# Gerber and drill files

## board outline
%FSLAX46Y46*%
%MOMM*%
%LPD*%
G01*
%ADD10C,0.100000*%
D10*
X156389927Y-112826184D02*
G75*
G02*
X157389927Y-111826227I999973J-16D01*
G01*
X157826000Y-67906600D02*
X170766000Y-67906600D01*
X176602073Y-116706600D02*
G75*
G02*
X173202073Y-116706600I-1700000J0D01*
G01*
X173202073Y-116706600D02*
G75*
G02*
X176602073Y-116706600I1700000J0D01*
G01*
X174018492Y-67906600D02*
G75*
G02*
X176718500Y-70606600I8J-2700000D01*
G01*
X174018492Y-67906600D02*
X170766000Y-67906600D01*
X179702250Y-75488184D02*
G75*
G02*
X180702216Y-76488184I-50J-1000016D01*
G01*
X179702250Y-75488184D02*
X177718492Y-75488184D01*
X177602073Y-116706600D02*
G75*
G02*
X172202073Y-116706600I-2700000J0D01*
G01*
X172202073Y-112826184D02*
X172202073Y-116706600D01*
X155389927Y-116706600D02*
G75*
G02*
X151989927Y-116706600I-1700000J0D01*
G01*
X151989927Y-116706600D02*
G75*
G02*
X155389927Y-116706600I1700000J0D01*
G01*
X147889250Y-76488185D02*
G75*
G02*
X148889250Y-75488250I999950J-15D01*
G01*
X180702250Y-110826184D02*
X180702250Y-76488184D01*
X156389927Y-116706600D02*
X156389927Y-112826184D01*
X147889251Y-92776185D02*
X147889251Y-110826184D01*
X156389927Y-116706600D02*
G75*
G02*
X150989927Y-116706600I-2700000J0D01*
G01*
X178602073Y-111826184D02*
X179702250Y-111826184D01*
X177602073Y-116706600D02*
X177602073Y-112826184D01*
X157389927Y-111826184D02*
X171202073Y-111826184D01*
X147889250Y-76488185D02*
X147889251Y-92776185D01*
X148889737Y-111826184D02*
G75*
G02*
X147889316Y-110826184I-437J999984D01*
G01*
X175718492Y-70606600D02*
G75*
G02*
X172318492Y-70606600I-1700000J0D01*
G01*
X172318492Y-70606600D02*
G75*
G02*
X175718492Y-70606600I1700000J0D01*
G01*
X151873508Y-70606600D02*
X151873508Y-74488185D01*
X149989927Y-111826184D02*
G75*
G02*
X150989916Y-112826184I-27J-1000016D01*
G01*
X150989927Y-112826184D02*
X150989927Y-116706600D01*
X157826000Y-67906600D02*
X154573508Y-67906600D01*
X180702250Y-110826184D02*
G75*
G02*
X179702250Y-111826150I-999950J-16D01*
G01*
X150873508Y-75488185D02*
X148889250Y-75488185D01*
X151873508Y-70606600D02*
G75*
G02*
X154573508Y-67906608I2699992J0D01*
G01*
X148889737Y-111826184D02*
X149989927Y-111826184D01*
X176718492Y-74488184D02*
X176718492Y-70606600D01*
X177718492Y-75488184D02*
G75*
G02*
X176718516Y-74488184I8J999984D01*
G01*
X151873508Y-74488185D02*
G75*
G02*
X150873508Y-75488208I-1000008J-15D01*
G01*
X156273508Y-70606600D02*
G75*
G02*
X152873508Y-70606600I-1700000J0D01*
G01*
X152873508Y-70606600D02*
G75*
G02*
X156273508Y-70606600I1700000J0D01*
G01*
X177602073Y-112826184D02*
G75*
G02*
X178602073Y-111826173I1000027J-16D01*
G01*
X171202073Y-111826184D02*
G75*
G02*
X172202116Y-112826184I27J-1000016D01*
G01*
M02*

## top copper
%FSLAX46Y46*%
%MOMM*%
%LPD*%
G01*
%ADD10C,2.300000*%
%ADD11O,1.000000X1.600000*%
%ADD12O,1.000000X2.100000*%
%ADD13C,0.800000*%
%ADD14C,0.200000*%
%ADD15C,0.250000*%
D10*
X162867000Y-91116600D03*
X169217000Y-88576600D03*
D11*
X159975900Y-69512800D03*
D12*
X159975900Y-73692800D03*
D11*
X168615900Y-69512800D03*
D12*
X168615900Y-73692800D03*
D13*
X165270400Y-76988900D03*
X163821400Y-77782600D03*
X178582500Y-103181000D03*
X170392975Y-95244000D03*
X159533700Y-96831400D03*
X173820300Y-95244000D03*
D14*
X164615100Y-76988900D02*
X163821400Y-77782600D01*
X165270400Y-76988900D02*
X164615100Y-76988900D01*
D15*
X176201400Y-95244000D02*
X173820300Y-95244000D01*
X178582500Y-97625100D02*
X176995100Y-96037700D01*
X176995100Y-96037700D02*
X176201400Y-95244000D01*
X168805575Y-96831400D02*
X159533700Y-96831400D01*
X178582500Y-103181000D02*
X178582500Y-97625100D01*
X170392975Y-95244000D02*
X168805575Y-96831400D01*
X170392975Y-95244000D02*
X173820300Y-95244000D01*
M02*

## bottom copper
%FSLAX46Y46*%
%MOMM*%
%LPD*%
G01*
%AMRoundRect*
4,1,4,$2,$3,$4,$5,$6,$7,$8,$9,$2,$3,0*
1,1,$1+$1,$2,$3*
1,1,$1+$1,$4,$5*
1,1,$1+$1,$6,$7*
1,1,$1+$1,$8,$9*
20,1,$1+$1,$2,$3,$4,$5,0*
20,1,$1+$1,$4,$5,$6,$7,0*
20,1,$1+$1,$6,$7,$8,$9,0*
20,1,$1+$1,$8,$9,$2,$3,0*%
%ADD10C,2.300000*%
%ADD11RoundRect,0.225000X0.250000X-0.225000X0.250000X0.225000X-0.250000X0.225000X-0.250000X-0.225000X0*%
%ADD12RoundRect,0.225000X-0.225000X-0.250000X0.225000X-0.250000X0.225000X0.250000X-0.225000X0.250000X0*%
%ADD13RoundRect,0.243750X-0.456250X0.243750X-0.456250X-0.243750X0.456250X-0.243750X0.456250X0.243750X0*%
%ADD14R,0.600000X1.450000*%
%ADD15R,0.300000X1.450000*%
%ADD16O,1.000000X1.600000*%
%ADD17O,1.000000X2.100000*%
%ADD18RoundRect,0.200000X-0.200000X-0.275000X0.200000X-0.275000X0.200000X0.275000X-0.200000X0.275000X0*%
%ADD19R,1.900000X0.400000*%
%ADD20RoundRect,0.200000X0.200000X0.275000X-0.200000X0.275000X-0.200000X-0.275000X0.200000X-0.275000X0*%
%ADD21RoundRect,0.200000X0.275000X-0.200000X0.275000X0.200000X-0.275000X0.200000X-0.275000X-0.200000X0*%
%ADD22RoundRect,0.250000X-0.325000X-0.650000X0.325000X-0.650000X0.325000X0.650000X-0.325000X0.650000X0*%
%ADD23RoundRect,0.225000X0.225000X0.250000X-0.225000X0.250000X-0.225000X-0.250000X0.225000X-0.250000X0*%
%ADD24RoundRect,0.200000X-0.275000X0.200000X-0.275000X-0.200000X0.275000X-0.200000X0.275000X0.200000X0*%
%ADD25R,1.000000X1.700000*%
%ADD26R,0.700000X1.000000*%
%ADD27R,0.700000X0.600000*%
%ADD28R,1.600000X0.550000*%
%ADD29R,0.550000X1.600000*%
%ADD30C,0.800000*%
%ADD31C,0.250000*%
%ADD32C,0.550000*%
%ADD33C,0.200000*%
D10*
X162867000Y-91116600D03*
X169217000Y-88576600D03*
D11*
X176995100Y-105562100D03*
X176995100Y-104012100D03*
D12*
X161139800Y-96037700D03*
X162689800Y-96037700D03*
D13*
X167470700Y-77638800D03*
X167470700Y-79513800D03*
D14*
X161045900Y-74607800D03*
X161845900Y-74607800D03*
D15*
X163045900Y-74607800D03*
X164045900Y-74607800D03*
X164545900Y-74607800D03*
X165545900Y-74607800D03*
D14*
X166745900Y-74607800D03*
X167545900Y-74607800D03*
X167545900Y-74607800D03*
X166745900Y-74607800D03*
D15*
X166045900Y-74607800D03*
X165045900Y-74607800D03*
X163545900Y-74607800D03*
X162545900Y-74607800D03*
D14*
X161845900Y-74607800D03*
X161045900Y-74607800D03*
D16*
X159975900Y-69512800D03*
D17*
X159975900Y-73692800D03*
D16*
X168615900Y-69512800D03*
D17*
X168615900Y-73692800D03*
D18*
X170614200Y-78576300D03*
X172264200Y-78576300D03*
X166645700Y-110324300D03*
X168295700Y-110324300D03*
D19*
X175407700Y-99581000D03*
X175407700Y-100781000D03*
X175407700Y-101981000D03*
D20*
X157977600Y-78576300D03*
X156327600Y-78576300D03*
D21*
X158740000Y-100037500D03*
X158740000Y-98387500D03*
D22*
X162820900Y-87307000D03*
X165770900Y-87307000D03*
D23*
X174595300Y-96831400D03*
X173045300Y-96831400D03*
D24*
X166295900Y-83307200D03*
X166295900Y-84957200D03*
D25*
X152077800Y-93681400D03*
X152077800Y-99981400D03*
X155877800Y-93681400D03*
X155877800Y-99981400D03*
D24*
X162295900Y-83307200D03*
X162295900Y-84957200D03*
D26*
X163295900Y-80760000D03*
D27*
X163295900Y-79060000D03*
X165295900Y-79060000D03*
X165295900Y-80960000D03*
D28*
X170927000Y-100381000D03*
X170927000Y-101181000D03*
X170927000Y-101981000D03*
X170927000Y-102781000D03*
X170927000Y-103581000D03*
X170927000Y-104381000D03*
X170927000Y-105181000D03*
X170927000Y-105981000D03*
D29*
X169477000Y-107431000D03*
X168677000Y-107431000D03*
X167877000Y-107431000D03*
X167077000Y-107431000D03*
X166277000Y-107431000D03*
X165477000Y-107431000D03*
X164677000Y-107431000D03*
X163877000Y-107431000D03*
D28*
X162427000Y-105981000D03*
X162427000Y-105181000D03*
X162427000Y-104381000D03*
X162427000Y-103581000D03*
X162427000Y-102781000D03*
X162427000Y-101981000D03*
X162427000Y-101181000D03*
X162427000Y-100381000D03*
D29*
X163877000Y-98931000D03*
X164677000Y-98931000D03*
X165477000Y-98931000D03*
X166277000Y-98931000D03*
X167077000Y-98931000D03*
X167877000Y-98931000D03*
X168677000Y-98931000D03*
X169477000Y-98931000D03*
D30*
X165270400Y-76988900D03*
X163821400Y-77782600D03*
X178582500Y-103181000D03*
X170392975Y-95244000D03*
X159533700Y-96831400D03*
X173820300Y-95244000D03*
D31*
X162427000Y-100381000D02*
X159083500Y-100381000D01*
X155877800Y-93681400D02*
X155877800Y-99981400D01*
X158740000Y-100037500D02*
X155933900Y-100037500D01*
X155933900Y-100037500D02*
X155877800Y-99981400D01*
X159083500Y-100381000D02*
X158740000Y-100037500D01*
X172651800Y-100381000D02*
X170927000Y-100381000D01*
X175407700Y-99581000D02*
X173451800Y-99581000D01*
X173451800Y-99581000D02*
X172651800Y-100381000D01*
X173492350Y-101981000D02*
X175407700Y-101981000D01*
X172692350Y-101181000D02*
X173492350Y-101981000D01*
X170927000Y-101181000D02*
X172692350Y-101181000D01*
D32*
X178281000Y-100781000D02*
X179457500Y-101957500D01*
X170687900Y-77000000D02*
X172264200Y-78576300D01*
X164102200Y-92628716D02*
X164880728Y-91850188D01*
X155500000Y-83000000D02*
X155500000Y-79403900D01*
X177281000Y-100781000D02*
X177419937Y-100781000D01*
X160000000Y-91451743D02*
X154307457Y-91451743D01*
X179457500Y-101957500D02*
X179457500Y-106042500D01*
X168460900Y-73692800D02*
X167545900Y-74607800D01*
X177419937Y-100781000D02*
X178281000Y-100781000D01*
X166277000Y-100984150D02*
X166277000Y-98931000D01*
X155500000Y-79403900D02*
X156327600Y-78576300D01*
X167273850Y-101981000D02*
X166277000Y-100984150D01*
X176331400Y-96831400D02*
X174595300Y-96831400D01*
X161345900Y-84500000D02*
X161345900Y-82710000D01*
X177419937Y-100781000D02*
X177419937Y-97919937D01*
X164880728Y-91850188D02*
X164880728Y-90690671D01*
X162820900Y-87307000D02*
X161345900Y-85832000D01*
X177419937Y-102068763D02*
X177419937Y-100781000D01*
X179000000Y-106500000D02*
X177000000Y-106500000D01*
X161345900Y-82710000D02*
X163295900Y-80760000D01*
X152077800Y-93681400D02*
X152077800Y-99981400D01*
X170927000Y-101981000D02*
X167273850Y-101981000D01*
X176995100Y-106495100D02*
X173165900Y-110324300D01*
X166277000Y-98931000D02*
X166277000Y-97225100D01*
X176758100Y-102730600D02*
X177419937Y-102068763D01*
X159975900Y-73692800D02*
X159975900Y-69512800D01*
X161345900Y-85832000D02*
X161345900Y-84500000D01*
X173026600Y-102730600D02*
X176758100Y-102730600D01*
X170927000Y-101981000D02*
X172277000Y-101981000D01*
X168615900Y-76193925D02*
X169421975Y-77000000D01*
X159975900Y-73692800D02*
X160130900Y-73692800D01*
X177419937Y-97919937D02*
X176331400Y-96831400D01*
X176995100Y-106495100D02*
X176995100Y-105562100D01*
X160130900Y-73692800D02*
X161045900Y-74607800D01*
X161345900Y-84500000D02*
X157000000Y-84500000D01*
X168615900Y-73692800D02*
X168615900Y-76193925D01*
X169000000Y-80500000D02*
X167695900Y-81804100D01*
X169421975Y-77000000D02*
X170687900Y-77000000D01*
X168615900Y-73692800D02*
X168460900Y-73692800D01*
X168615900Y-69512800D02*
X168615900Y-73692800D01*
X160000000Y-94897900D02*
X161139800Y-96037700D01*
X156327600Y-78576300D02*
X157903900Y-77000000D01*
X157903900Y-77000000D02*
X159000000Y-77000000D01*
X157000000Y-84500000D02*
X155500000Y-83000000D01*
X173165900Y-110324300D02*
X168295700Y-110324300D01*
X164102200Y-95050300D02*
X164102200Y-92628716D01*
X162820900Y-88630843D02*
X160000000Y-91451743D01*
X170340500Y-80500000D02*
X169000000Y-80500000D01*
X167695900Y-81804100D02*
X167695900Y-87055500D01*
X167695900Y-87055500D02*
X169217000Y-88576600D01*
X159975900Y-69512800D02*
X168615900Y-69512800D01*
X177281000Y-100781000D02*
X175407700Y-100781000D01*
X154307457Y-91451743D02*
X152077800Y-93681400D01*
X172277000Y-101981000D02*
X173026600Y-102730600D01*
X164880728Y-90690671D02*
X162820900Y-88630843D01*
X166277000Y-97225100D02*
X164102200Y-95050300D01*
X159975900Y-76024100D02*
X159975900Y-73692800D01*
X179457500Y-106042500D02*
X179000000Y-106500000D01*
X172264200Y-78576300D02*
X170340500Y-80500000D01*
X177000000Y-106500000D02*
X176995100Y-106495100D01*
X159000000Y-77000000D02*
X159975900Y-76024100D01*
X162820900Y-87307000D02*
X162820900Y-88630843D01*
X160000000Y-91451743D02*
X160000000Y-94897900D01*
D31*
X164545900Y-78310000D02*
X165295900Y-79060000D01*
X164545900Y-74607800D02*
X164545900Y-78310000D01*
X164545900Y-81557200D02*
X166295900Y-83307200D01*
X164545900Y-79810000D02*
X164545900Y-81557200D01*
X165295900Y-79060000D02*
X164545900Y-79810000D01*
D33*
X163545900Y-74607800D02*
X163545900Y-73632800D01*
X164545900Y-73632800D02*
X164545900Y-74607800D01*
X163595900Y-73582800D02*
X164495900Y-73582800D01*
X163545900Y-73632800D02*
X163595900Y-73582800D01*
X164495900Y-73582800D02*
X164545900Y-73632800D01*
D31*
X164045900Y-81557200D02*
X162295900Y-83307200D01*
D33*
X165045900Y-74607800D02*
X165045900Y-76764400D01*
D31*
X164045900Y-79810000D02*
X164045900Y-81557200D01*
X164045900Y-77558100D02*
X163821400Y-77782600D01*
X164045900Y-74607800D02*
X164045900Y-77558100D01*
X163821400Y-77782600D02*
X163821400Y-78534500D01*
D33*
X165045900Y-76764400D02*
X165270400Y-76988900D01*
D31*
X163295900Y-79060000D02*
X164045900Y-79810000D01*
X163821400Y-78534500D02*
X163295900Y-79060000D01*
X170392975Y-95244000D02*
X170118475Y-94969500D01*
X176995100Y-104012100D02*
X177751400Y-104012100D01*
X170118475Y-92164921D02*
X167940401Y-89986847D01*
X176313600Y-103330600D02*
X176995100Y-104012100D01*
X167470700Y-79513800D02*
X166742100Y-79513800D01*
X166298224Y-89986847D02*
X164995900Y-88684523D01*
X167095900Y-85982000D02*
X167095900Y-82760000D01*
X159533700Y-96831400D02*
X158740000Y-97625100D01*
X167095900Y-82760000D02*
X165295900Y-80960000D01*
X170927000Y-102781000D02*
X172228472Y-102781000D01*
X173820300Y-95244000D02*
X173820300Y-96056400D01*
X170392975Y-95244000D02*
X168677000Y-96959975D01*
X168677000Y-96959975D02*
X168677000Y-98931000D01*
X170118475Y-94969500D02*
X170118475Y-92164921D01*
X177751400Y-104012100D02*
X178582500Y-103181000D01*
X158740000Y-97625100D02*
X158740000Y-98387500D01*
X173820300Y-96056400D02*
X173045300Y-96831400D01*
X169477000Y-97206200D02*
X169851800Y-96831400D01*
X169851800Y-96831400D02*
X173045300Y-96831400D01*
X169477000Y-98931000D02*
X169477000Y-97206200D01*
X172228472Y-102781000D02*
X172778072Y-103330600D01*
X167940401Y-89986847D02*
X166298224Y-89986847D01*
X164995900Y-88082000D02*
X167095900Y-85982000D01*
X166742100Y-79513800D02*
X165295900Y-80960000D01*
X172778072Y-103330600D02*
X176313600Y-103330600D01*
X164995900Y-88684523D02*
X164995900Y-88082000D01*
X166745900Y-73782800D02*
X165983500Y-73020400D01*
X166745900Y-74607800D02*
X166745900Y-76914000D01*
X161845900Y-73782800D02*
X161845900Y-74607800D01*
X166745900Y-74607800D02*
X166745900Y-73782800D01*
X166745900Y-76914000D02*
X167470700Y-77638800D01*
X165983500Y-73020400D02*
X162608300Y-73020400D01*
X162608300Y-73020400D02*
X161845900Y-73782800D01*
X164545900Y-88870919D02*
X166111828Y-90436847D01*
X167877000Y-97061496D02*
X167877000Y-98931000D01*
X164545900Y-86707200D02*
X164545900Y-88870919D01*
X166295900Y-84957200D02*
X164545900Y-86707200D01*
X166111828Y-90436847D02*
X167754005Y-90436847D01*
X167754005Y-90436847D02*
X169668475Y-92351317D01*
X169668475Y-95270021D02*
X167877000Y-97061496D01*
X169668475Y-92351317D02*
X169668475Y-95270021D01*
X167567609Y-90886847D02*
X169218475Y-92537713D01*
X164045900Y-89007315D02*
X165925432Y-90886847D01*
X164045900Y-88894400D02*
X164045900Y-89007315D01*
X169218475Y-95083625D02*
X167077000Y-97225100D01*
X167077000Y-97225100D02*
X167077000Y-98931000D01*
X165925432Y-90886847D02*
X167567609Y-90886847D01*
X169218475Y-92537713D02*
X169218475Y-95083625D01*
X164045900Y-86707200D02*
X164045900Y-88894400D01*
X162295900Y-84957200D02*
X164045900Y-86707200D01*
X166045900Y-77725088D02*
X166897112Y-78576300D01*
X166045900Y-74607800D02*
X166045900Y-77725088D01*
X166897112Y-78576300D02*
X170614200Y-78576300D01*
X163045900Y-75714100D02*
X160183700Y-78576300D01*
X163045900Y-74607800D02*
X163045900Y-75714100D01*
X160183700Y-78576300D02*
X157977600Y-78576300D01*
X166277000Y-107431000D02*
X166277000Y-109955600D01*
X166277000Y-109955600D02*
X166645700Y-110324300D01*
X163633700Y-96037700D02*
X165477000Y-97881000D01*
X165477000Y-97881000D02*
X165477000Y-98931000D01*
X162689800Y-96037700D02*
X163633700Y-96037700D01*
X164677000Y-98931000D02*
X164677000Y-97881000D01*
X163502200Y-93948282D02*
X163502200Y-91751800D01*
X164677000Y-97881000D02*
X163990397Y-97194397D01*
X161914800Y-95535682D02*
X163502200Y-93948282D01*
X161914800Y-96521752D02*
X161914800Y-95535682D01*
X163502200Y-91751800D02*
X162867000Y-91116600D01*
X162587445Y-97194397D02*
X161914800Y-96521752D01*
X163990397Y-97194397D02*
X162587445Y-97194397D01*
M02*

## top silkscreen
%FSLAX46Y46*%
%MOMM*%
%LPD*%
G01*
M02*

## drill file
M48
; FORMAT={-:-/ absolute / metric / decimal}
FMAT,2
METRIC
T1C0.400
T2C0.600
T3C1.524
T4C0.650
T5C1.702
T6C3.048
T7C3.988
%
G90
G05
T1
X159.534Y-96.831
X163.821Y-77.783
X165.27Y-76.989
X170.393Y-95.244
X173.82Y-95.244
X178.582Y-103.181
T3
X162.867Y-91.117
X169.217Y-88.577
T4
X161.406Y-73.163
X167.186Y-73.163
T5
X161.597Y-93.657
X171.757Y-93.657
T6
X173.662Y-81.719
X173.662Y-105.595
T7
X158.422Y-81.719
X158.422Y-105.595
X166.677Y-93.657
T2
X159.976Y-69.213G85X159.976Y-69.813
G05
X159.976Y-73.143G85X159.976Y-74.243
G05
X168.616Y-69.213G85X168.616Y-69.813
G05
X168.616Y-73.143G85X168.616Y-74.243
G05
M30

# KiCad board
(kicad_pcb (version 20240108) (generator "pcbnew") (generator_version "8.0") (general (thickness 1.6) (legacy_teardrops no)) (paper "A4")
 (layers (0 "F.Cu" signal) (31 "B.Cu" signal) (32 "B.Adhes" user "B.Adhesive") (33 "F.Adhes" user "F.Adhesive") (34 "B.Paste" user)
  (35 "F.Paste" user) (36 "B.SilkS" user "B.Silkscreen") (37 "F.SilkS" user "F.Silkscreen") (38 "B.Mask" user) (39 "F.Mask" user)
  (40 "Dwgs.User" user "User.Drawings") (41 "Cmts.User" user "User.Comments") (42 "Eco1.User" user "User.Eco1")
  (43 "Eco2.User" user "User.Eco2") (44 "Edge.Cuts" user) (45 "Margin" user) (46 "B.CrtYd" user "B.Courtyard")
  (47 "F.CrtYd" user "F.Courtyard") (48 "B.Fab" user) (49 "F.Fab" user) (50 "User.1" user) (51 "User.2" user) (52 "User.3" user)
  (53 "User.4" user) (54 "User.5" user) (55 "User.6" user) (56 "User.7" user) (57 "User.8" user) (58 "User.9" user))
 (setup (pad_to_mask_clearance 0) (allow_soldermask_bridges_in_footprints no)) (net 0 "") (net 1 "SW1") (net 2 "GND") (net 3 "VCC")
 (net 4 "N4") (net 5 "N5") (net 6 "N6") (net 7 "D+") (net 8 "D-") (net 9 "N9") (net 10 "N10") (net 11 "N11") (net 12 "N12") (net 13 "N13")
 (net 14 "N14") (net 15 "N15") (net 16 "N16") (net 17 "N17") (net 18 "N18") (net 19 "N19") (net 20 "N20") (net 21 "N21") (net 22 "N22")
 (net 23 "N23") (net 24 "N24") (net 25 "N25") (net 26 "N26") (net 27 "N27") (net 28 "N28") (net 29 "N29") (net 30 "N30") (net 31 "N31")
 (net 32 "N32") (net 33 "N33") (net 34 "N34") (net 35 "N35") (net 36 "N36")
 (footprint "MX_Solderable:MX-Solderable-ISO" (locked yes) (layer "F.Cu") (at 166.677 93.6566)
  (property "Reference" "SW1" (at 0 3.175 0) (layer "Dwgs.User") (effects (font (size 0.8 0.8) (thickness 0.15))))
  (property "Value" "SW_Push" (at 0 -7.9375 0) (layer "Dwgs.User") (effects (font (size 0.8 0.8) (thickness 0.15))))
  (pad "" np_thru_hole circle (at -8.255 -11.938) (size 3.9878 3.9878) (drill 3.9878) (layers "*.Cu" "*.Mask"))
  (pad "" np_thru_hole circle (at -8.255 11.938) (size 3.9878 3.9878) (drill 3.9878) (layers "*.Cu" "*.Mask"))
  (pad "" np_thru_hole circle (at -5.08 0 48.099) (size 1.7018 1.7018) (drill 1.7018) (layers "F&B.Cu" "*.Mask"))
  (pad "" np_thru_hole circle (at 0 0) (size 3.9878 3.9878) (drill 3.9878) (layers "*.Cu" "*.Mask"))
  (pad "" np_thru_hole circle (at 5.08 0 48.099) (size 1.7018 1.7018) (drill 1.7018) (layers "F&B.Cu" "*.Mask"))
  (pad "" np_thru_hole circle (at 6.985 -11.938) (size 3.048 3.048) (drill 3.048) (layers "*.Cu" "*.Mask"))
  (pad "" np_thru_hole circle (at 6.985 11.938) (size 3.048 3.048) (drill 3.048) (layers "*.Cu" "*.Mask"))
  (pad "1" thru_hole circle (at -3.81 -2.54) (size 2.3 2.3) (drill 1.524) (layers "*.Cu" "B.Mask") (remove_unused_layers no) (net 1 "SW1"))
  (pad "2" thru_hole circle (at 2.54 -5.08) (size 2.3 2.3) (drill 1.524) (layers "*.Cu" "B.Mask") (remove_unused_layers no) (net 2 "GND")))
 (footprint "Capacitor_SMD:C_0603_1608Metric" (layer "B.Cu") (at 176.9951 104.7871 90)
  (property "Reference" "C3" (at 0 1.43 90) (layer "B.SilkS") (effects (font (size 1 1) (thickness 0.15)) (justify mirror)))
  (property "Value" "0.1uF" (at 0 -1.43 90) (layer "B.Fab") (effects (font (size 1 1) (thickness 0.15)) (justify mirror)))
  (pad "1" smd roundrect (at -0.775 0 90) (size 0.9 0.95) (layers "B.Cu" "B.Paste" "B.Mask") (roundrect_rratio 0.25) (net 2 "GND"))
  (pad "2" smd roundrect (at 0.775 0 90) (size 0.9 0.95) (layers "B.Cu" "B.Paste" "B.Mask") (roundrect_rratio 0.25) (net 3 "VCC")))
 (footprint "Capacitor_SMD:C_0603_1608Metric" (layer "B.Cu") (at 161.9148 96.0377)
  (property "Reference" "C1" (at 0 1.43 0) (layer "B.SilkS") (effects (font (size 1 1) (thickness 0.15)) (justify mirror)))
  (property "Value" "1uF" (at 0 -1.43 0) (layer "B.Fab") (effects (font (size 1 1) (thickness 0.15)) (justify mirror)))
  (pad "1" smd roundrect (at -0.775 0) (size 0.9 0.95) (layers "B.Cu" "B.Paste" "B.Mask") (roundrect_rratio 0.25) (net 2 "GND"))
  (pad "2" smd roundrect (at 0.775 0) (size 0.9 0.95) (layers "B.Cu" "B.Paste" "B.Mask") (roundrect_rratio 0.25) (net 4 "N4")))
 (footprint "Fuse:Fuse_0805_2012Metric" (layer "B.Cu") (at 167.4707 78.5763 -90)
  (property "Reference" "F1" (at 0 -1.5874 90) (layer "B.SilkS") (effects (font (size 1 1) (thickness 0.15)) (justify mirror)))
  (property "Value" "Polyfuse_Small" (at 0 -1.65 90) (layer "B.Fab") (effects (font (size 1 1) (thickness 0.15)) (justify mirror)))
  (pad "1" smd roundrect (at -0.9375 0 270) (size 0.975 1.4) (layers "B.Cu" "B.Paste" "B.Mask") (roundrect_rratio 0.25) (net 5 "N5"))
  (pad "2" smd roundrect (at 0.9375 0 270) (size 0.975 1.4) (layers "B.Cu" "B.Paste" "B.Mask") (roundrect_rratio 0.25) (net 3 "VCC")))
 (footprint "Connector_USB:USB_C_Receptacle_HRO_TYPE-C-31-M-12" (layer "B.Cu") (at 164.2959 70.5628)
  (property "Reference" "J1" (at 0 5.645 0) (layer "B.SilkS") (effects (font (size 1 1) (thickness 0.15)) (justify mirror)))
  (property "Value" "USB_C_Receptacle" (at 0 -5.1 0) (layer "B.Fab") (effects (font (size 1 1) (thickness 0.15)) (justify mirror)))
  (pad "" np_thru_hole circle (at -2.89 2.6) (size 0.65 0.65) (drill 0.65) (layers "*.Cu" "*.Mask"))
  (pad "" np_thru_hole circle (at 2.89 2.6) (size 0.65 0.65) (drill 0.65) (layers "*.Cu" "*.Mask"))
  (pad "A1" smd rect (at -3.25 4.045) (size 0.6 1.45) (layers "B.Cu" "B.Paste" "B.Mask") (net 2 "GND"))
  (pad "A4" smd rect (at -2.45 4.045) (size 0.6 1.45) (layers "B.Cu" "B.Paste" "B.Mask") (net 5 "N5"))
  (pad "A5" smd rect (at -1.25 4.045) (size 0.3 1.45) (layers "B.Cu" "B.Paste" "B.Mask") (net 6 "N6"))
  (pad "A6" smd rect (at -0.25 4.045) (size 0.3 1.45) (layers "B.Cu" "B.Paste" "B.Mask") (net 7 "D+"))
  (pad "A7" smd rect (at 0.25 4.045) (size 0.3 1.45) (layers "B.Cu" "B.Paste" "B.Mask") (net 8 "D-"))
  (pad "A8" smd rect (at 1.25 4.045) (size 0.3 1.45) (layers "B.Cu" "B.Paste" "B.Mask") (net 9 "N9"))
  (pad "A9" smd rect (at 2.45 4.045) (size 0.6 1.45) (layers "B.Cu" "B.Paste" "B.Mask") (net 5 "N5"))
  (pad "A12" smd rect (at 3.25 4.045) (size 0.6 1.45) (layers "B.Cu" "B.Paste" "B.Mask") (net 2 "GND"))
  (pad "B1" smd rect (at 3.25 4.045) (size 0.6 1.45) (layers "B.Cu" "B.Paste" "B.Mask") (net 2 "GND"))
  (pad "B4" smd rect (at 2.45 4.045) (size 0.6 1.45) (layers "B.Cu" "B.Paste" "B.Mask") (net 5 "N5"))
  (pad "B5" smd rect (at 1.75 4.045) (size 0.3 1.45) (layers "B.Cu" "B.Paste" "B.Mask") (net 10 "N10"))
  (pad "B6" smd rect (at 0.75 4.045) (size 0.3 1.45) (layers "B.Cu" "B.Paste" "B.Mask") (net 7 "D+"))
  (pad "B7" smd rect (at -0.75 4.045) (size 0.3 1.45) (layers "B.Cu" "B.Paste" "B.Mask") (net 8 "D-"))
  (pad "B8" smd rect (at -1.75 4.045) (size 0.3 1.45) (layers "B.Cu" "B.Paste" "B.Mask") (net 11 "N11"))
  (pad "B9" smd rect (at -2.45 4.045) (size 0.6 1.45) (layers "B.Cu" "B.Paste" "B.Mask") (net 5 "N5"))
  (pad "B12" smd rect (at -3.25 4.045) (size 0.6 1.45) (layers "B.Cu" "B.Paste" "B.Mask") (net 2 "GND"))
  (pad "S1" thru_hole oval (at -4.32 -1.05) (size 1 1.6) (drill oval 0.6 1.2) (layers "*.Cu" "*.Mask") (remove_unused_layers no)
   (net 2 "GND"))
  (pad "S1" thru_hole oval (at -4.32 3.13) (size 1 2.1) (drill oval 0.6 1.7) (layers "*.Cu" "*.Mask") (remove_unused_layers no)
   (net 2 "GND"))
  (pad "S1" thru_hole oval (at 4.32 -1.05) (size 1 1.6) (drill oval 0.6 1.2) (layers "*.Cu" "*.Mask") (remove_unused_layers no)
   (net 2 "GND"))
  (pad "S1" thru_hole oval (at 4.32 3.13) (size 1 2.1) (drill oval 0.6 1.7) (layers "*.Cu" "*.Mask") (remove_unused_layers no) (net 2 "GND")))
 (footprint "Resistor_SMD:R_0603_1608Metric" (layer "B.Cu") (at 171.4392 78.5763)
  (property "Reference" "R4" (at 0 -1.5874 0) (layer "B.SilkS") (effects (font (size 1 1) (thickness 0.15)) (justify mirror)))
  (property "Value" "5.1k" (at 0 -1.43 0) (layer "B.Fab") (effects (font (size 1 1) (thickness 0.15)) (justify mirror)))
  (pad "1" smd roundrect (at -0.825 0) (size 0.8 0.95) (layers "B.Cu" "B.Paste" "B.Mask") (roundrect_rratio 0.25) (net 10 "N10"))
  (pad "2" smd roundrect (at 0.825 0) (size 0.8 0.95) (layers "B.Cu" "B.Paste" "B.Mask") (roundrect_rratio 0.25) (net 2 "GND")))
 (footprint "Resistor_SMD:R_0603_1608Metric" (layer "B.Cu") (at 167.4707 110.3243)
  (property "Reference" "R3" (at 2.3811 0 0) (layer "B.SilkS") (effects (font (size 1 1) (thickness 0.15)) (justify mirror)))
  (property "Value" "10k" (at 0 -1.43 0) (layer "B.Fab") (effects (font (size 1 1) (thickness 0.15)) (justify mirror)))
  (pad "1" smd roundrect (at -0.825 0) (size 0.8 0.95) (layers "B.Cu" "B.Paste" "B.Mask") (roundrect_rratio 0.25) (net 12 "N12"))
  (pad "2" smd roundrect (at 0.825 0) (size 0.8 0.95) (layers "B.Cu" "B.Paste" "B.Mask") (roundrect_rratio 0.25) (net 2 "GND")))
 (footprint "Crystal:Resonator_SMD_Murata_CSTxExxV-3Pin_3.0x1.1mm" (layer "B.Cu") (at 175.4077 100.781 -90)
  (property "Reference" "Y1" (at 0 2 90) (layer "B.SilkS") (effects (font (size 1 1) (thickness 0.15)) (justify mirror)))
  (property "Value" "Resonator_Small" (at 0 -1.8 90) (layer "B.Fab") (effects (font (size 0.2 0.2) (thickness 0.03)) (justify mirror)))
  (pad "1" smd rect (at -1.2 0 270) (size 0.4 1.9) (layers "B.Cu" "B.Paste" "B.Mask") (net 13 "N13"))
  (pad "2" smd rect (at 0 0 270) (size 0.4 1.9) (layers "B.Cu" "B.Paste" "B.Mask") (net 2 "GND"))
  (pad "3" smd rect (at 1.2 0 270) (size 0.4 1.9) (layers "B.Cu" "B.Paste" "B.Mask") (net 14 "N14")))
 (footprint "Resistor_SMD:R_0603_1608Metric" (layer "B.Cu") (at 157.1526 78.5763 180)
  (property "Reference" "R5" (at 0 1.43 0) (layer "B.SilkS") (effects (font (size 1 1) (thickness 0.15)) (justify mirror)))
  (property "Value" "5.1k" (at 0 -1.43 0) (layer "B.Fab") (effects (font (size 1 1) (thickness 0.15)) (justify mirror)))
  (pad "1" smd roundrect (at -0.825 0 180) (size 0.8 0.95) (layers "B.Cu" "B.Paste" "B.Mask") (roundrect_rratio 0.25) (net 6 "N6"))
  (pad "2" smd roundrect (at 0.825 0 180) (size 0.8 0.95) (layers "B.Cu" "B.Paste" "B.Mask") (roundrect_rratio 0.25) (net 2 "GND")))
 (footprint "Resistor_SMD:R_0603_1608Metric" (layer "B.Cu") (at 158.74 99.2125 90)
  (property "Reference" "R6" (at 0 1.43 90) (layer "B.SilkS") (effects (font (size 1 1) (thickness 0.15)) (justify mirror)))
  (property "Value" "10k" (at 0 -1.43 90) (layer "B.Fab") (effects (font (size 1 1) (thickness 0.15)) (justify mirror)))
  (pad "1" smd roundrect (at -0.825 0 90) (size 0.8 0.95) (layers "B.Cu" "B.Paste" "B.Mask") (roundrect_rratio 0.25) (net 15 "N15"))
  (pad "2" smd roundrect (at 0.825 0 90) (size 0.8 0.95) (layers "B.Cu" "B.Paste" "B.Mask") (roundrect_rratio 0.25) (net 3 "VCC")))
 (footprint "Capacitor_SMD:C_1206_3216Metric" (layer "B.Cu") (at 164.2959 87.307)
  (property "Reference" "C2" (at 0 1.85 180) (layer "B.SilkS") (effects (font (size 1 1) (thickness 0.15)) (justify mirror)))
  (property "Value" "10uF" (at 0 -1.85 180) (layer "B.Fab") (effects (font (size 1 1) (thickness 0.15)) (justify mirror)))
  (pad "1" smd roundrect (at -1.475 0) (size 1.15 1.8) (layers "B.Cu" "B.Paste" "B.Mask") (roundrect_rratio 0.2173913043) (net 2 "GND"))
  (pad "2" smd roundrect (at 1.475 0) (size 1.15 1.8) (layers "B.Cu" "B.Paste" "B.Mask") (roundrect_rratio 0.2173913043) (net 3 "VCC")))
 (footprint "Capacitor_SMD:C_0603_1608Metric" (layer "B.Cu") (at 173.8203 96.8314 180)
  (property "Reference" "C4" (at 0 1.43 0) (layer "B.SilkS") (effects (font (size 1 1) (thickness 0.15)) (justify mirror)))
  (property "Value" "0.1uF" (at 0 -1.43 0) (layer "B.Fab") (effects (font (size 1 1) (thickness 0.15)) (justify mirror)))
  (pad "1" smd roundrect (at -0.775 0 180) (size 0.9 0.95) (layers "B.Cu" "B.Paste" "B.Mask") (roundrect_rratio 0.25) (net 2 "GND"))
  (pad "2" smd roundrect (at 0.775 0 180) (size 0.9 0.95) (layers "B.Cu" "B.Paste" "B.Mask") (roundrect_rratio 0.25) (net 3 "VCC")))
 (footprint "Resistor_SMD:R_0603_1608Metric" (layer "B.Cu") (at 166.2959 84.1322 -90)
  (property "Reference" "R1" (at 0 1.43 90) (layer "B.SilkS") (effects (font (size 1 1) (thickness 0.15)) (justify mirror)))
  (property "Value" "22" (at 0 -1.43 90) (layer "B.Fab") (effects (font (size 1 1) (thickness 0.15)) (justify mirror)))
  (pad "1" smd roundrect (at -0.825 0 270) (size 0.8 0.95) (layers "B.Cu" "B.Paste" "B.Mask") (roundrect_rratio 0.25) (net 8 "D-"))
  (pad "2" smd roundrect (at 0.825 0 270) (size 0.8 0.95) (layers "B.Cu" "B.Paste" "B.Mask") (roundrect_rratio 0.25) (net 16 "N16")))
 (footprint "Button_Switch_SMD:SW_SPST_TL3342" (layer "B.Cu") (at 153.9778 96.8314 -90)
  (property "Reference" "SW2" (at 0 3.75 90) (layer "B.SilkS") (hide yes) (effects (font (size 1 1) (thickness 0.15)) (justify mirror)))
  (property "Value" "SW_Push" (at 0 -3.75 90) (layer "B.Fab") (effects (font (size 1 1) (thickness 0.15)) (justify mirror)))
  (pad "1" smd rect (at -3.15 1.9 270) (size 1.7 1) (layers "B.Cu" "B.Paste" "B.Mask") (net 2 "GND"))
  (pad "1" smd rect (at 3.15 1.9 270) (size 1.7 1) (layers "B.Cu" "B.Paste" "B.Mask") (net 2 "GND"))
  (pad "2" smd rect (at -3.15 -1.9 270) (size 1.7 1) (layers "B.Cu" "B.Paste" "B.Mask") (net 15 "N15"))
  (pad "2" smd rect (at 3.15 -1.9 270) (size 1.7 1) (layers "B.Cu" "B.Paste" "B.Mask") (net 15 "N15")))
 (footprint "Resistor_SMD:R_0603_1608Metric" (layer "B.Cu") (at 162.2959 84.1322 -90)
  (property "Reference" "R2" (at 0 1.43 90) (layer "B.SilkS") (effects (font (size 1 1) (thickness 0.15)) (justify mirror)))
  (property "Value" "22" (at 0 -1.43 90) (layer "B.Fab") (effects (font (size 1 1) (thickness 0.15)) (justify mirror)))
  (pad "1" smd roundrect (at -0.825 0 270) (size 0.8 0.95) (layers "B.Cu" "B.Paste" "B.Mask") (roundrect_rratio 0.25) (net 7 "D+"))
  (pad "2" smd roundrect (at 0.825 0 270) (size 0.8 0.95) (layers "B.Cu" "B.Paste" "B.Mask") (roundrect_rratio 0.25) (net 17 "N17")))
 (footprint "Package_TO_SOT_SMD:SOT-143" (layer "B.Cu") (at 164.2959 80.01)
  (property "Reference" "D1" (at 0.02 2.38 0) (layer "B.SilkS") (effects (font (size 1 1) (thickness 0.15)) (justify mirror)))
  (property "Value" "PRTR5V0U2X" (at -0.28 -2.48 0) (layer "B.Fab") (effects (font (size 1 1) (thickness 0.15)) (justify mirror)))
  (pad "1" smd rect (at -1 0.75) (size 0.7 1) (layers "B.Cu" "B.Paste" "B.Mask") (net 2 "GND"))
  (pad "2" smd rect (at -1 -0.95) (size 0.7 0.6) (layers "B.Cu" "B.Paste" "B.Mask") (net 7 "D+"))
  (pad "3" smd rect (at 1 -0.95) (size 0.7 0.6) (layers "B.Cu" "B.Paste" "B.Mask") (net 8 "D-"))
  (pad "4" smd rect (at 1 0.95) (size 0.7 0.6) (layers "B.Cu" "B.Paste" "B.Mask") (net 3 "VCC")))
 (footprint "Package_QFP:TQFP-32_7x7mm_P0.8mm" (layer "B.Cu") (at 166.677 103.181 180)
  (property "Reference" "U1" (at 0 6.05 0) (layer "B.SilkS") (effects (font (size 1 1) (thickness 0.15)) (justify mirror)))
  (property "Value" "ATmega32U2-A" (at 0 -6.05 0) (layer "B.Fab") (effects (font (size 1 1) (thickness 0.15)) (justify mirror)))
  (pad "1" smd rect (at -4.25 2.8 180) (size 1.6 0.55) (layers "B.Cu" "B.Paste" "B.Mask") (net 13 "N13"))
  (pad "2" smd rect (at -4.25 2 180) (size 1.6 0.55) (layers "B.Cu" "B.Paste" "B.Mask") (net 14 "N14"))
  (pad "3" smd rect (at -4.25 1.2 180) (size 1.6 0.55) (layers "B.Cu" "B.Paste" "B.Mask") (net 2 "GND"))
  (pad "4" smd rect (at -4.25 0.4 180) (size 1.6 0.55) (layers "B.Cu" "B.Paste" "B.Mask") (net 3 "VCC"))
  (pad "5" smd rect (at -4.25 -0.4 180) (size 1.6 0.55) (layers "B.Cu" "B.Paste" "B.Mask") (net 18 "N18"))
  (pad "6" smd rect (at -4.25 -1.2 180) (size 1.6 0.55) (layers "B.Cu" "B.Paste" "B.Mask") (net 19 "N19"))
  (pad "7" smd rect (at -4.25 -2 180) (size 1.6 0.55) (layers "B.Cu" "B.Paste" "B.Mask") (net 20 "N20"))
  (pad "8" smd rect (at -4.25 -2.8 180) (size 1.6 0.55) (layers "B.Cu" "B.Paste" "B.Mask") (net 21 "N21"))
  (pad "9" smd rect (at -2.8 -4.25 90) (size 1.6 0.55) (layers "B.Cu" "B.Paste" "B.Mask") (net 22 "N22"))
  (pad "10" smd rect (at -2 -4.25 90) (size 1.6 0.55) (layers "B.Cu" "B.Paste" "B.Mask") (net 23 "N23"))
  (pad "11" smd rect (at -1.2 -4.25 90) (size 1.6 0.55) (layers "B.Cu" "B.Paste" "B.Mask") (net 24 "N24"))
  (pad "12" smd rect (at -0.4 -4.25 90) (size 1.6 0.55) (layers "B.Cu" "B.Paste" "B.Mask") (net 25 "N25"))
  (pad "13" smd rect (at 0.4 -4.25 90) (size 1.6 0.55) (layers "B.Cu" "B.Paste" "B.Mask") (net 12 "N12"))
  (pad "14" smd rect (at 1.2 -4.25 90) (size 1.6 0.55) (layers "B.Cu" "B.Paste" "B.Mask") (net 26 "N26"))
  (pad "15" smd rect (at 2 -4.25 90) (size 1.6 0.55) (layers "B.Cu" "B.Paste" "B.Mask") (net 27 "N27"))
  (pad "16" smd rect (at 2.8 -4.25 90) (size 1.6 0.55) (layers "B.Cu" "B.Paste" "B.Mask") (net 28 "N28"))
  (pad "17" smd rect (at 4.25 -2.8 180) (size 1.6 0.55) (layers "B.Cu" "B.Paste" "B.Mask") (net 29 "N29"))
  (pad "18" smd rect (at 4.25 -2 180) (size 1.6 0.55) (layers "B.Cu" "B.Paste" "B.Mask") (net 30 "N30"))
  (pad "19" smd rect (at 4.25 -1.2 180) (size 1.6 0.55) (layers "B.Cu" "B.Paste" "B.Mask") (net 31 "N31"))
  (pad "20" smd rect (at 4.25 -0.4 180) (size 1.6 0.55) (layers "B.Cu" "B.Paste" "B.Mask") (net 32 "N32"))
  (pad "21" smd rect (at 4.25 0.4 180) (size 1.6 0.55) (layers "B.Cu" "B.Paste" "B.Mask") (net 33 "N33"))
  (pad "22" smd rect (at 4.25 1.2 180) (size 1.6 0.55) (layers "B.Cu" "B.Paste" "B.Mask") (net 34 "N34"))
  (pad "23" smd rect (at 4.25 2 180) (size 1.6 0.55) (layers "B.Cu" "B.Paste" "B.Mask") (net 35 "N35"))
  (pad "24" smd rect (at 4.25 2.8 180) (size 1.6 0.55) (layers "B.Cu" "B.Paste" "B.Mask") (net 15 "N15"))
  (pad "25" smd rect (at 2.8 4.25 90) (size 1.6 0.55) (layers "B.Cu" "B.Paste" "B.Mask") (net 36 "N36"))
  (pad "26" smd rect (at 2 4.25 90) (size 1.6 0.55) (layers "B.Cu" "B.Paste" "B.Mask") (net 1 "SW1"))
  (pad "27" smd rect (at 1.2 4.25 90) (size 1.6 0.55) (layers "B.Cu" "B.Paste" "B.Mask") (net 4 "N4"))
  (pad "28" smd rect (at 0.4 4.25 90) (size 1.6 0.55) (layers "B.Cu" "B.Paste" "B.Mask") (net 2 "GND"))
  (pad "29" smd rect (at -0.4 4.25 90) (size 1.6 0.55) (layers "B.Cu" "B.Paste" "B.Mask") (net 17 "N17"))
  (pad "30" smd rect (at -1.2 4.25 90) (size 1.6 0.55) (layers "B.Cu" "B.Paste" "B.Mask") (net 16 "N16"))
  (pad "31" smd rect (at -2 4.25 90) (size 1.6 0.55) (layers "B.Cu" "B.Paste" "B.Mask") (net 3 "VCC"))
  (pad "32" smd rect (at -2.8 4.25 90) (size 1.6 0.55) (layers "B.Cu" "B.Paste" "B.Mask") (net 3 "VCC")))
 (gr_arc (start 156.389927 112.826184) (mid 156.682821 112.119078) (end 157.389927 111.826184) (stroke (width 0.1) (type solid))
  (layer "Edge.Cuts"))
 (gr_line (start 157.826 67.9066) (end 170.766 67.9066) (stroke (width 0.1) (type default)) (layer "Edge.Cuts"))
 (gr_circle (center 174.902073 116.7066) (end 173.202073 116.7066) (stroke (width 0.1) (type solid)) (fill none) (layer "Edge.Cuts"))
 (gr_arc (start 174.018492 67.9066) (mid 175.92768 68.697412) (end 176.718492 70.6066) (stroke (width 0.1) (type solid)) (layer "Edge.Cuts"))
 (gr_line (start 174.018492 67.9066) (end 170.766 67.9066) (stroke (width 0.1) (type solid)) (layer "Edge.Cuts"))
 (gr_arc (start 179.70225 75.488184) (mid 180.409356 75.781078) (end 180.70225 76.488184) (stroke (width 0.1) (type solid))
  (layer "Edge.Cuts"))
 (gr_line (start 179.70225 75.488184) (end 177.718492 75.488184) (stroke (width 0.1) (type solid)) (layer "Edge.Cuts"))
 (gr_arc (start 177.602073 116.7066) (mid 174.902073 119.4066) (end 172.202073 116.7066) (stroke (width 0.1) (type solid))
  (layer "Edge.Cuts"))
 (gr_line (start 172.202073 112.826184) (end 172.202073 116.7066) (stroke (width 0.1) (type solid)) (layer "Edge.Cuts"))
 (gr_circle (center 153.689927 116.7066) (end 151.989927 116.7066) (stroke (width 0.1) (type solid)) (fill none) (layer "Edge.Cuts"))
 (gr_arc (start 147.88925 76.488185) (mid 148.182141 75.781075) (end 148.88925 75.488185) (stroke (width 0.1) (type solid))
  (layer "Edge.Cuts"))
 (gr_line (start 180.70225 110.826184) (end 180.70225 76.488184) (stroke (width 0.1) (type solid)) (layer "Edge.Cuts"))
 (gr_line (start 156.389927 116.7066) (end 156.389927 112.826184) (stroke (width 0.1) (type solid)) (layer "Edge.Cuts"))
 (gr_line (start 147.889251 92.776185) (end 147.889251 110.826184) (stroke (width 0.1) (type solid)) (layer "Edge.Cuts"))
 (gr_arc (start 156.389927 116.7066) (mid 153.689927 119.4066) (end 150.989927 116.7066) (stroke (width 0.1) (type solid))
  (layer "Edge.Cuts"))
 (gr_line (start 178.602073 111.826184) (end 179.70225 111.826184) (stroke (width 0.1) (type solid)) (layer "Edge.Cuts"))
 (gr_line (start 177.602073 116.7066) (end 177.602073 112.826184) (stroke (width 0.1) (type solid)) (layer "Edge.Cuts"))
 (gr_line (start 157.389927 111.826184) (end 171.202073 111.826184) (stroke (width 0.1) (type solid)) (layer "Edge.Cuts"))
 (gr_line (start 147.88925 76.488185) (end 147.889251 92.776185) (stroke (width 0.1) (type solid)) (layer "Edge.Cuts"))
 (gr_arc (start 148.889737 111.826184) (mid 148.182316 111.533463) (end 147.889251 110.826184) (stroke (width 0.1) (type solid))
  (layer "Edge.Cuts"))
 (gr_circle (center 174.018492 70.6066) (end 172.318492 70.6066) (stroke (width 0.1) (type solid)) (fill none) (layer "Edge.Cuts"))
 (gr_line (start 151.873508 70.6066) (end 151.873508 74.488185) (stroke (width 0.1) (type solid)) (layer "Edge.Cuts"))
 (gr_arc (start 149.989927 111.826184) (mid 150.697033 112.119078) (end 150.989927 112.826184) (stroke (width 0.1) (type solid))
  (layer "Edge.Cuts"))
 (gr_line (start 150.989927 112.826184) (end 150.989927 116.7066) (stroke (width 0.1) (type solid)) (layer "Edge.Cuts"))
 (gr_line (start 157.826 67.9066) (end 154.573508 67.9066) (stroke (width 0.1) (type solid)) (layer "Edge.Cuts"))
 (gr_arc (start 180.70225 110.826184) (mid 180.409357 111.533291) (end 179.70225 111.826184) (stroke (width 0.1) (type solid))
  (layer "Edge.Cuts"))
 (gr_line (start 150.873508 75.488185) (end 148.88925 75.488185) (stroke (width 0.1) (type solid)) (layer "Edge.Cuts"))
 (gr_arc (start 151.873508 70.6066) (mid 152.66432 68.697412) (end 154.573508 67.9066) (stroke (width 0.1) (type solid)) (layer "Edge.Cuts"))
 (gr_line (start 148.889737 111.826184) (end 149.989927 111.826184) (stroke (width 0.1) (type solid)) (layer "Edge.Cuts"))
 (gr_line (start 176.718492 74.488184) (end 176.718492 70.6066) (stroke (width 0.1) (type solid)) (layer "Edge.Cuts"))
 (gr_arc (start 177.718492 75.488184) (mid 177.011385 75.195291) (end 176.718492 74.488184) (stroke (width 0.1) (type solid))
  (layer "Edge.Cuts"))
 (gr_arc (start 151.873508 74.488185) (mid 151.580614 75.195291) (end 150.873508 75.488185) (stroke (width 0.1) (type solid))
  (layer "Edge.Cuts"))
 (gr_circle (center 154.573508 70.6066) (end 152.873508 70.6066) (stroke (width 0.1) (type solid)) (fill none) (layer "Edge.Cuts"))
 (gr_arc (start 177.602073 112.826184) (mid 177.894967 112.119078) (end 178.602073 111.826184) (stroke (width 0.1) (type solid))
  (layer "Edge.Cuts"))
 (gr_arc (start 171.202073 111.826184) (mid 171.909179 112.119078) (end 172.202073 112.826184) (stroke (width 0.1) (type solid))
  (layer "Edge.Cuts"))
 (segment (start 162.427 100.381) (end 159.0835 100.381) (width 0.25) (layer "B.Cu") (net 15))
 (segment (start 155.8778 93.6814) (end 155.8778 99.9814) (width 0.25) (layer "B.Cu") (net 15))
 (segment (start 158.74 100.0375) (end 155.9339 100.0375) (width 0.25) (layer "B.Cu") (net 15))
 (segment (start 155.9339 100.0375) (end 155.8778 99.9814) (width 0.25) (layer "B.Cu") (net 15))
 (segment (start 159.0835 100.381) (end 158.74 100.0375) (width 0.25) (layer "B.Cu") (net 15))
 (segment (start 172.6518 100.381) (end 170.927 100.381) (width 0.25) (layer "B.Cu") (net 13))
 (segment (start 175.4077 99.581) (end 173.4518 99.581) (width 0.25) (layer "B.Cu") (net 13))
 (segment (start 173.4518 99.581) (end 172.6518 100.381) (width 0.25) (layer "B.Cu") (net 13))
 (segment (start 173.49235 101.981) (end 175.4077 101.981) (width 0.25) (layer "B.Cu") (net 14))
 (segment (start 172.69235 101.181) (end 173.49235 101.981) (width 0.25) (layer "B.Cu") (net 14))
 (segment (start 170.927 101.181) (end 172.69235 101.181) (width 0.25) (layer "B.Cu") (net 14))
 (segment (start 178.281 100.781) (end 179.4575 101.9575) (width 0.55) (layer "B.Cu") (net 2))
 (segment (start 170.6879 77) (end 172.2642 78.5763) (width 0.55) (layer "B.Cu") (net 2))
 (segment (start 164.1022 92.628716) (end 164.880728 91.850188) (width 0.55) (layer "B.Cu") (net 2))
 (segment (start 155.5 83) (end 155.5 79.4039) (width 0.55) (layer "B.Cu") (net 2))
 (segment (start 177.281 100.781) (end 177.419937 100.781) (width 0.55) (layer "B.Cu") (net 2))
 (segment (start 160 91.451743) (end 154.307457 91.451743) (width 0.55) (layer "B.Cu") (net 2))
 (segment (start 179.4575 101.9575) (end 179.4575 106.0425) (width 0.55) (layer "B.Cu") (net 2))
 (segment (start 168.4609 73.6928) (end 167.5459 74.6078) (width 0.55) (layer "B.Cu") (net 2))
 (segment (start 177.419937 100.781) (end 178.281 100.781) (width 0.55) (layer "B.Cu") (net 2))
 (segment (start 166.277 100.98415) (end 166.277 98.931) (width 0.55) (layer "B.Cu") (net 2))
 (segment (start 155.5 79.4039) (end 156.3276 78.5763) (width 0.55) (layer "B.Cu") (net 2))
 (segment (start 167.27385 101.981) (end 166.277 100.98415) (width 0.55) (layer "B.Cu") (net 2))
 (segment (start 176.3314 96.8314) (end 174.5953 96.8314) (width 0.55) (layer "B.Cu") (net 2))
 (segment (start 161.3459 84.5) (end 161.3459 82.71) (width 0.55) (layer "B.Cu") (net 2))
 (segment (start 177.419937 100.781) (end 177.419937 97.919937) (width 0.55) (layer "B.Cu") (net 2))
 (segment (start 164.880728 91.850188) (end 164.880728 90.690671) (width 0.55) (layer "B.Cu") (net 2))
 (segment (start 162.8209 87.307) (end 161.3459 85.832) (width 0.55) (layer "B.Cu") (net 2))
 (segment (start 177.419937 102.068763) (end 177.419937 100.781) (width 0.55) (layer "B.Cu") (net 2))
 (segment (start 179 106.5) (end 177 106.5) (width 0.55) (layer "B.Cu") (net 2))
 (segment (start 161.3459 82.71) (end 163.2959 80.76) (width 0.55) (layer "B.Cu") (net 2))
 (segment (start 152.0778 93.6814) (end 152.0778 99.9814) (width 0.55) (layer "B.Cu") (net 2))
 (segment (start 170.927 101.981) (end 167.27385 101.981) (width 0.55) (layer "B.Cu") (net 2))
 (segment (start 176.9951 106.4951) (end 173.1659 110.3243) (width 0.55) (layer "B.Cu") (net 2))
 (segment (start 166.277 98.931) (end 166.277 97.2251) (width 0.55) (layer "B.Cu") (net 2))
 (segment (start 176.7581 102.7306) (end 177.419937 102.068763) (width 0.55) (layer "B.Cu") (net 2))
 (segment (start 159.9759 73.6928) (end 159.9759 69.5128) (width 0.55) (layer "B.Cu") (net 2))
 (segment (start 161.3459 85.832) (end 161.3459 84.5) (width 0.55) (layer "B.Cu") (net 2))
 (segment (start 173.0266 102.7306) (end 176.7581 102.7306) (width 0.55) (layer "B.Cu") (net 2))
 (segment (start 170.927 101.981) (end 172.277 101.981) (width 0.55) (layer "B.Cu") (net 2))
 (segment (start 168.6159 76.193925) (end 169.421975 77) (width 0.55) (layer "B.Cu") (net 2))
 (segment (start 159.9759 73.6928) (end 160.1309 73.6928) (width 0.55) (layer "B.Cu") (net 2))
 (segment (start 177.419937 97.919937) (end 176.3314 96.8314) (width 0.55) (layer "B.Cu") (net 2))
 (segment (start 176.9951 106.4951) (end 176.9951 105.5621) (width 0.55) (layer "B.Cu") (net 2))
 (segment (start 160.1309 73.6928) (end 161.0459 74.6078) (width 0.55) (layer "B.Cu") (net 2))
 (segment (start 161.3459 84.5) (end 157 84.5) (width 0.55) (layer "B.Cu") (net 2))
 (segment (start 168.6159 73.6928) (end 168.6159 76.193925) (width 0.55) (layer "B.Cu") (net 2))
 (segment (start 169 80.5) (end 167.6959 81.8041) (width 0.55) (layer "B.Cu") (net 2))
 (segment (start 169.421975 77) (end 170.6879 77) (width 0.55) (layer "B.Cu") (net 2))
 (segment (start 168.6159 73.6928) (end 168.4609 73.6928) (width 0.55) (layer "B.Cu") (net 2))
 (segment (start 168.6159 69.5128) (end 168.6159 73.6928) (width 0.55) (layer "B.Cu") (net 2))
 (segment (start 160 94.8979) (end 161.1398 96.0377) (width 0.55) (layer "B.Cu") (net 2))
 (segment (start 156.3276 78.5763) (end 157.9039 77) (width 0.55) (layer "B.Cu") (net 2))
 (segment (start 157.9039 77) (end 159 77) (width 0.55) (layer "B.Cu") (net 2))
 (segment (start 157 84.5) (end 155.5 83) (width 0.55) (layer "B.Cu") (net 2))
 (segment (start 173.1659 110.3243) (end 168.2957 110.3243) (width 0.55) (layer "B.Cu") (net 2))
 (segment (start 164.1022 95.0503) (end 164.1022 92.628716) (width 0.55) (layer "B.Cu") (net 2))
 (segment (start 162.8209 88.630843) (end 160 91.451743) (width 0.55) (layer "B.Cu") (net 2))
 (segment (start 170.3405 80.5) (end 169 80.5) (width 0.55) (layer "B.Cu") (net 2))
 (segment (start 167.6959 81.8041) (end 167.6959 87.0555) (width 0.55) (layer "B.Cu") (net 2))
 (segment (start 167.6959 87.0555) (end 169.217 88.5766) (width 0.55) (layer "B.Cu") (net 2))
 (segment (start 159.9759 69.5128) (end 168.6159 69.5128) (width 0.55) (layer "B.Cu") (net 2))
 (segment (start 177.281 100.781) (end 175.4077 100.781) (width 0.55) (layer "B.Cu") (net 2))
 (segment (start 154.307457 91.451743) (end 152.0778 93.6814) (width 0.55) (layer "B.Cu") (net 2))
 (segment (start 172.277 101.981) (end 173.0266 102.7306) (width 0.55) (layer "B.Cu") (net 2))
 (segment (start 164.880728 90.690671) (end 162.8209 88.630843) (width 0.55) (layer "B.Cu") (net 2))
 (segment (start 166.277 97.2251) (end 164.1022 95.0503) (width 0.55) (layer "B.Cu") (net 2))
 (segment (start 159.9759 76.0241) (end 159.9759 73.6928) (width 0.55) (layer "B.Cu") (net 2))
 (segment (start 179.4575 106.0425) (end 179 106.5) (width 0.55) (layer "B.Cu") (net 2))
 (segment (start 172.2642 78.5763) (end 170.3405 80.5) (width 0.55) (layer "B.Cu") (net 2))
 (segment (start 177 106.5) (end 176.9951 106.4951) (width 0.55) (layer "B.Cu") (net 2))
 (segment (start 159 77) (end 159.9759 76.0241) (width 0.55) (layer "B.Cu") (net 2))
 (segment (start 162.8209 87.307) (end 162.8209 88.630843) (width 0.55) (layer "B.Cu") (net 2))
 (segment (start 160 91.451743) (end 160 94.8979) (width 0.55) (layer "B.Cu") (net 2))
 (segment (start 164.5459 78.31) (end 165.2959 79.06) (width 0.25) (layer "B.Cu") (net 8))
 (segment (start 164.5459 74.6078) (end 164.5459 78.31) (width 0.25) (layer "B.Cu") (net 8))
 (segment (start 164.5459 81.5572) (end 166.2959 83.3072) (width 0.25) (layer "B.Cu") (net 8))
 (segment (start 164.5459 79.81) (end 164.5459 81.5572) (width 0.25) (layer "B.Cu") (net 8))
 (segment (start 165.2959 79.06) (end 164.5459 79.81) (width 0.25) (layer "B.Cu") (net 8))
 (segment (start 163.5459 74.6078) (end 163.5459 73.6328) (width 0.2) (layer "B.Cu") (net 8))
 (segment (start 164.5459 73.6328) (end 164.5459 74.6078) (width 0.2) (layer "B.Cu") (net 8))
 (segment (start 163.5959 73.5828) (end 164.4959 73.5828) (width 0.2) (layer "B.Cu") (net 8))
 (segment (start 163.5459 73.6328) (end 163.5959 73.5828) (width 0.2) (layer "B.Cu") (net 8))
 (segment (start 164.4959 73.5828) (end 164.5459 73.6328) (width 0.2) (layer "B.Cu") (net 8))
 (segment (start 164.6151 76.9889) (end 163.8214 77.7826) (width 0.2) (layer "F.Cu") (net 7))
 (segment (start 165.2704 76.9889) (end 164.6151 76.9889) (width 0.2) (layer "F.Cu") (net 7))
 (via (at 165.2704 76.9889) (size 0.8) (drill 0.4) (layers "F.Cu" "B.Cu") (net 7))
 (via (at 163.8214 77.7826) (size 0.8) (drill 0.4) (layers "F.Cu" "B.Cu") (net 7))
 (segment (start 164.0459 81.5572) (end 162.2959 83.3072) (width 0.25) (layer "B.Cu") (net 7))
 (segment (start 165.0459 74.6078) (end 165.0459 76.7644) (width 0.2) (layer "B.Cu") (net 7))
 (segment (start 164.0459 79.81) (end 164.0459 81.5572) (width 0.25) (layer "B.Cu") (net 7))
 (segment (start 164.0459 77.5581) (end 163.8214 77.7826) (width 0.25) (layer "B.Cu") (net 7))
 (segment (start 164.0459 74.6078) (end 164.0459 77.5581) (width 0.25) (layer "B.Cu") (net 7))
 (segment (start 163.8214 77.7826) (end 163.8214 78.5345) (width 0.25) (layer "B.Cu") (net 7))
 (segment (start 165.0459 76.7644) (end 165.2704 76.9889) (width 0.2) (layer "B.Cu") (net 7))
 (segment (start 163.2959 79.06) (end 164.0459 79.81) (width 0.25) (layer "B.Cu") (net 7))
 (segment (start 163.8214 78.5345) (end 163.2959 79.06) (width 0.25) (layer "B.Cu") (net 7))
 (segment (start 176.2014 95.244) (end 173.8203 95.244) (width 0.25) (layer "F.Cu") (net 3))
 (segment (start 178.5825 97.6251) (end 176.9951 96.0377) (width 0.25) (layer "F.Cu") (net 3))
 (segment (start 176.9951 96.0377) (end 176.2014 95.244) (width 0.25) (layer "F.Cu") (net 3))
 (segment (start 168.805575 96.8314) (end 159.5337 96.8314) (width 0.25) (layer "F.Cu") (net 3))
 (segment (start 178.5825 103.181) (end 178.5825 97.6251) (width 0.25) (layer "F.Cu") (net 3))
 (segment (start 170.392975 95.244) (end 168.805575 96.8314) (width 0.25) (layer "F.Cu") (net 3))
 (segment (start 170.392975 95.244) (end 173.8203 95.244) (width 0.25) (layer "F.Cu") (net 3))
 (via (at 178.5825 103.181) (size 0.8) (drill 0.4) (layers "F.Cu" "B.Cu") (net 3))
 (via (at 170.392975 95.244) (size 0.8) (drill 0.4) (layers "F.Cu" "B.Cu") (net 3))
 (via (at 159.5337 96.8314) (size 0.8) (drill 0.4) (layers "F.Cu" "B.Cu") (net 3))
 (via (at 173.8203 95.244) (size 0.8) (drill 0.4) (layers "F.Cu" "B.Cu") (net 3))
 (segment (start 170.392975 95.244) (end 170.118475 94.9695) (width 0.25) (layer "B.Cu") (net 3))
 (segment (start 176.9951 104.0121) (end 177.7514 104.0121) (width 0.25) (layer "B.Cu") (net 3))
 (segment (start 170.118475 92.164921) (end 167.940401 89.986847) (width 0.25) (layer "B.Cu") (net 3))
 (segment (start 176.3136 103.3306) (end 176.9951 104.0121) (width 0.25) (layer "B.Cu") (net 3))
 (segment (start 167.4707 79.5138) (end 166.7421 79.5138) (width 0.25) (layer "B.Cu") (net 3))
 (segment (start 166.298224 89.986847) (end 164.9959 88.684523) (width 0.25) (layer "B.Cu") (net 3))
 (segment (start 167.0959 85.982) (end 167.0959 82.76) (width 0.25) (layer "B.Cu") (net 3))
 (segment (start 159.5337 96.8314) (end 158.74 97.6251) (width 0.25) (layer "B.Cu") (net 3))
 (segment (start 167.0959 82.76) (end 165.2959 80.96) (width 0.25) (layer "B.Cu") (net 3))
 (segment (start 170.927 102.781) (end 172.228472 102.781) (width 0.25) (layer "B.Cu") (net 3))
 (segment (start 173.8203 95.244) (end 173.8203 96.0564) (width 0.25) (layer "B.Cu") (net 3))
 (segment (start 170.392975 95.244) (end 168.677 96.959975) (width 0.25) (layer "B.Cu") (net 3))
 (segment (start 168.677 96.959975) (end 168.677 98.931) (width 0.25) (layer "B.Cu") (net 3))
 (segment (start 170.118475 94.9695) (end 170.118475 92.164921) (width 0.25) (layer "B.Cu") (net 3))
 (segment (start 177.7514 104.0121) (end 178.5825 103.181) (width 0.25) (layer "B.Cu") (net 3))
 (segment (start 158.74 97.6251) (end 158.74 98.3875) (width 0.25) (layer "B.Cu") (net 3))
 (segment (start 173.8203 96.0564) (end 173.0453 96.8314) (width 0.25) (layer "B.Cu") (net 3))
 (segment (start 169.477 97.2062) (end 169.8518 96.8314) (width 0.25) (layer "B.Cu") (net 3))
 (segment (start 169.8518 96.8314) (end 173.0453 96.8314) (width 0.25) (layer "B.Cu") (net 3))
 (segment (start 169.477 98.931) (end 169.477 97.2062) (width 0.25) (layer "B.Cu") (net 3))
 (segment (start 172.228472 102.781) (end 172.778072 103.3306) (width 0.25) (layer "B.Cu") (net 3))
 (segment (start 167.940401 89.986847) (end 166.298224 89.986847) (width 0.25) (layer "B.Cu") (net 3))
 (segment (start 164.9959 88.082) (end 167.0959 85.982) (width 0.25) (layer "B.Cu") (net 3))
 (segment (start 166.7421 79.5138) (end 165.2959 80.96) (width 0.25) (layer "B.Cu") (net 3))
 (segment (start 172.778072 103.3306) (end 176.3136 103.3306) (width 0.25) (layer "B.Cu") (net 3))
 (segment (start 164.9959 88.684523) (end 164.9959 88.082) (width 0.25) (layer "B.Cu") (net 3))
 (segment (start 166.7459 73.7828) (end 165.9835 73.0204) (width 0.25) (layer "B.Cu") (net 5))
 (segment (start 166.7459 74.6078) (end 166.7459 76.914) (width 0.25) (layer "B.Cu") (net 5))
 (segment (start 161.8459 73.7828) (end 161.8459 74.6078) (width 0.25) (layer "B.Cu") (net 5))
 (segment (start 166.7459 74.6078) (end 166.7459 73.7828) (width 0.25) (layer "B.Cu") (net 5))
 (segment (start 166.7459 76.914) (end 167.4707 77.6388) (width 0.25) (layer "B.Cu") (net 5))
 (segment (start 165.9835 73.0204) (end 162.6083 73.0204) (width 0.25) (layer "B.Cu") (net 5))
 (segment (start 162.6083 73.0204) (end 161.8459 73.7828) (width 0.25) (layer "B.Cu") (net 5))
 (segment (start 164.5459 88.870919) (end 166.111828 90.436847) (width 0.25) (layer "B.Cu") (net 16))
 (segment (start 167.877 97.061496) (end 167.877 98.931) (width 0.25) (layer "B.Cu") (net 16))
 (segment (start 164.5459 86.7072) (end 164.5459 88.870919) (width 0.25) (layer "B.Cu") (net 16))
 (segment (start 166.2959 84.9572) (end 164.5459 86.7072) (width 0.25) (layer "B.Cu") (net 16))
 (segment (start 166.111828 90.436847) (end 167.754005 90.436847) (width 0.25) (layer "B.Cu") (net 16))
 (segment (start 167.754005 90.436847) (end 169.668475 92.351317) (width 0.25) (layer "B.Cu") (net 16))
 (segment (start 169.668475 95.270021) (end 167.877 97.061496) (width 0.25) (layer "B.Cu") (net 16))
 (segment (start 169.668475 92.351317) (end 169.668475 95.270021) (width 0.25) (layer "B.Cu") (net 16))
 (segment (start 167.567609 90.886847) (end 169.218475 92.537713) (width 0.25) (layer "B.Cu") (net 17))
 (segment (start 164.0459 89.007315) (end 165.925432 90.886847) (width 0.25) (layer "B.Cu") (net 17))
 (segment (start 164.0459 88.8944) (end 164.0459 89.007315) (width 0.25) (layer "B.Cu") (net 17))
 (segment (start 169.218475 95.083625) (end 167.077 97.2251) (width 0.25) (layer "B.Cu") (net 17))
 (segment (start 167.077 97.2251) (end 167.077 98.931) (width 0.25) (layer "B.Cu") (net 17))
 (segment (start 165.925432 90.886847) (end 167.567609 90.886847) (width 0.25) (layer "B.Cu") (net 17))
 (segment (start 169.218475 92.537713) (end 169.218475 95.083625) (width 0.25) (layer "B.Cu") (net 17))
 (segment (start 164.0459 86.7072) (end 164.0459 88.8944) (width 0.25) (layer "B.Cu") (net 17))
 (segment (start 162.2959 84.9572) (end 164.0459 86.7072) (width 0.25) (layer "B.Cu") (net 17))
 (segment (start 166.0459 77.725088) (end 166.897112 78.5763) (width 0.25) (layer "B.Cu") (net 10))
 (segment (start 166.0459 74.6078) (end 166.0459 77.725088) (width 0.25) (layer "B.Cu") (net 10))
 (segment (start 166.897112 78.5763) (end 170.6142 78.5763) (width 0.25) (layer "B.Cu") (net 10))
 (segment (start 163.0459 75.7141) (end 160.1837 78.5763) (width 0.25) (layer "B.Cu") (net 6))
 (segment (start 163.0459 74.6078) (end 163.0459 75.7141) (width 0.25) (layer "B.Cu") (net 6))
 (segment (start 160.1837 78.5763) (end 157.9776 78.5763) (width 0.25) (layer "B.Cu") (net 6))
 (segment (start 166.277 107.431) (end 166.277 109.9556) (width 0.25) (layer "B.Cu") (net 12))
 (segment (start 166.277 109.9556) (end 166.6457 110.3243) (width 0.25) (layer "B.Cu") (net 12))
 (segment (start 163.6337 96.0377) (end 165.477 97.881) (width 0.25) (layer "B.Cu") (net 4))
 (segment (start 165.477 97.881) (end 165.477 98.931) (width 0.25) (layer "B.Cu") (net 4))
 (segment (start 162.6898 96.0377) (end 163.6337 96.0377) (width 0.25) (layer "B.Cu") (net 4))
 (segment (start 164.677 98.931) (end 164.677 97.881) (width 0.25) (layer "B.Cu") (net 1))
 (segment (start 163.5022 93.948282) (end 163.5022 91.7518) (width 0.25) (layer "B.Cu") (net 1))
 (segment (start 164.677 97.881) (end 163.990397 97.194397) (width 0.25) (layer "B.Cu") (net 1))
 (segment (start 161.9148 95.535682) (end 163.5022 93.948282) (width 0.25) (layer "B.Cu") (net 1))
 (segment (start 161.9148 96.521752) (end 161.9148 95.535682) (width 0.25) (layer "B.Cu") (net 1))
 (segment (start 163.5022 91.7518) (end 162.867 91.1166) (width 0.25) (layer "B.Cu") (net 1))
 (segment (start 162.587445 97.194397) (end 161.9148 96.521752) (width 0.25) (layer "B.Cu") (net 1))
 (segment (start 163.990397 97.194397) (end 162.587445 97.194397) (width 0.25) (layer "B.Cu") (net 1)))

